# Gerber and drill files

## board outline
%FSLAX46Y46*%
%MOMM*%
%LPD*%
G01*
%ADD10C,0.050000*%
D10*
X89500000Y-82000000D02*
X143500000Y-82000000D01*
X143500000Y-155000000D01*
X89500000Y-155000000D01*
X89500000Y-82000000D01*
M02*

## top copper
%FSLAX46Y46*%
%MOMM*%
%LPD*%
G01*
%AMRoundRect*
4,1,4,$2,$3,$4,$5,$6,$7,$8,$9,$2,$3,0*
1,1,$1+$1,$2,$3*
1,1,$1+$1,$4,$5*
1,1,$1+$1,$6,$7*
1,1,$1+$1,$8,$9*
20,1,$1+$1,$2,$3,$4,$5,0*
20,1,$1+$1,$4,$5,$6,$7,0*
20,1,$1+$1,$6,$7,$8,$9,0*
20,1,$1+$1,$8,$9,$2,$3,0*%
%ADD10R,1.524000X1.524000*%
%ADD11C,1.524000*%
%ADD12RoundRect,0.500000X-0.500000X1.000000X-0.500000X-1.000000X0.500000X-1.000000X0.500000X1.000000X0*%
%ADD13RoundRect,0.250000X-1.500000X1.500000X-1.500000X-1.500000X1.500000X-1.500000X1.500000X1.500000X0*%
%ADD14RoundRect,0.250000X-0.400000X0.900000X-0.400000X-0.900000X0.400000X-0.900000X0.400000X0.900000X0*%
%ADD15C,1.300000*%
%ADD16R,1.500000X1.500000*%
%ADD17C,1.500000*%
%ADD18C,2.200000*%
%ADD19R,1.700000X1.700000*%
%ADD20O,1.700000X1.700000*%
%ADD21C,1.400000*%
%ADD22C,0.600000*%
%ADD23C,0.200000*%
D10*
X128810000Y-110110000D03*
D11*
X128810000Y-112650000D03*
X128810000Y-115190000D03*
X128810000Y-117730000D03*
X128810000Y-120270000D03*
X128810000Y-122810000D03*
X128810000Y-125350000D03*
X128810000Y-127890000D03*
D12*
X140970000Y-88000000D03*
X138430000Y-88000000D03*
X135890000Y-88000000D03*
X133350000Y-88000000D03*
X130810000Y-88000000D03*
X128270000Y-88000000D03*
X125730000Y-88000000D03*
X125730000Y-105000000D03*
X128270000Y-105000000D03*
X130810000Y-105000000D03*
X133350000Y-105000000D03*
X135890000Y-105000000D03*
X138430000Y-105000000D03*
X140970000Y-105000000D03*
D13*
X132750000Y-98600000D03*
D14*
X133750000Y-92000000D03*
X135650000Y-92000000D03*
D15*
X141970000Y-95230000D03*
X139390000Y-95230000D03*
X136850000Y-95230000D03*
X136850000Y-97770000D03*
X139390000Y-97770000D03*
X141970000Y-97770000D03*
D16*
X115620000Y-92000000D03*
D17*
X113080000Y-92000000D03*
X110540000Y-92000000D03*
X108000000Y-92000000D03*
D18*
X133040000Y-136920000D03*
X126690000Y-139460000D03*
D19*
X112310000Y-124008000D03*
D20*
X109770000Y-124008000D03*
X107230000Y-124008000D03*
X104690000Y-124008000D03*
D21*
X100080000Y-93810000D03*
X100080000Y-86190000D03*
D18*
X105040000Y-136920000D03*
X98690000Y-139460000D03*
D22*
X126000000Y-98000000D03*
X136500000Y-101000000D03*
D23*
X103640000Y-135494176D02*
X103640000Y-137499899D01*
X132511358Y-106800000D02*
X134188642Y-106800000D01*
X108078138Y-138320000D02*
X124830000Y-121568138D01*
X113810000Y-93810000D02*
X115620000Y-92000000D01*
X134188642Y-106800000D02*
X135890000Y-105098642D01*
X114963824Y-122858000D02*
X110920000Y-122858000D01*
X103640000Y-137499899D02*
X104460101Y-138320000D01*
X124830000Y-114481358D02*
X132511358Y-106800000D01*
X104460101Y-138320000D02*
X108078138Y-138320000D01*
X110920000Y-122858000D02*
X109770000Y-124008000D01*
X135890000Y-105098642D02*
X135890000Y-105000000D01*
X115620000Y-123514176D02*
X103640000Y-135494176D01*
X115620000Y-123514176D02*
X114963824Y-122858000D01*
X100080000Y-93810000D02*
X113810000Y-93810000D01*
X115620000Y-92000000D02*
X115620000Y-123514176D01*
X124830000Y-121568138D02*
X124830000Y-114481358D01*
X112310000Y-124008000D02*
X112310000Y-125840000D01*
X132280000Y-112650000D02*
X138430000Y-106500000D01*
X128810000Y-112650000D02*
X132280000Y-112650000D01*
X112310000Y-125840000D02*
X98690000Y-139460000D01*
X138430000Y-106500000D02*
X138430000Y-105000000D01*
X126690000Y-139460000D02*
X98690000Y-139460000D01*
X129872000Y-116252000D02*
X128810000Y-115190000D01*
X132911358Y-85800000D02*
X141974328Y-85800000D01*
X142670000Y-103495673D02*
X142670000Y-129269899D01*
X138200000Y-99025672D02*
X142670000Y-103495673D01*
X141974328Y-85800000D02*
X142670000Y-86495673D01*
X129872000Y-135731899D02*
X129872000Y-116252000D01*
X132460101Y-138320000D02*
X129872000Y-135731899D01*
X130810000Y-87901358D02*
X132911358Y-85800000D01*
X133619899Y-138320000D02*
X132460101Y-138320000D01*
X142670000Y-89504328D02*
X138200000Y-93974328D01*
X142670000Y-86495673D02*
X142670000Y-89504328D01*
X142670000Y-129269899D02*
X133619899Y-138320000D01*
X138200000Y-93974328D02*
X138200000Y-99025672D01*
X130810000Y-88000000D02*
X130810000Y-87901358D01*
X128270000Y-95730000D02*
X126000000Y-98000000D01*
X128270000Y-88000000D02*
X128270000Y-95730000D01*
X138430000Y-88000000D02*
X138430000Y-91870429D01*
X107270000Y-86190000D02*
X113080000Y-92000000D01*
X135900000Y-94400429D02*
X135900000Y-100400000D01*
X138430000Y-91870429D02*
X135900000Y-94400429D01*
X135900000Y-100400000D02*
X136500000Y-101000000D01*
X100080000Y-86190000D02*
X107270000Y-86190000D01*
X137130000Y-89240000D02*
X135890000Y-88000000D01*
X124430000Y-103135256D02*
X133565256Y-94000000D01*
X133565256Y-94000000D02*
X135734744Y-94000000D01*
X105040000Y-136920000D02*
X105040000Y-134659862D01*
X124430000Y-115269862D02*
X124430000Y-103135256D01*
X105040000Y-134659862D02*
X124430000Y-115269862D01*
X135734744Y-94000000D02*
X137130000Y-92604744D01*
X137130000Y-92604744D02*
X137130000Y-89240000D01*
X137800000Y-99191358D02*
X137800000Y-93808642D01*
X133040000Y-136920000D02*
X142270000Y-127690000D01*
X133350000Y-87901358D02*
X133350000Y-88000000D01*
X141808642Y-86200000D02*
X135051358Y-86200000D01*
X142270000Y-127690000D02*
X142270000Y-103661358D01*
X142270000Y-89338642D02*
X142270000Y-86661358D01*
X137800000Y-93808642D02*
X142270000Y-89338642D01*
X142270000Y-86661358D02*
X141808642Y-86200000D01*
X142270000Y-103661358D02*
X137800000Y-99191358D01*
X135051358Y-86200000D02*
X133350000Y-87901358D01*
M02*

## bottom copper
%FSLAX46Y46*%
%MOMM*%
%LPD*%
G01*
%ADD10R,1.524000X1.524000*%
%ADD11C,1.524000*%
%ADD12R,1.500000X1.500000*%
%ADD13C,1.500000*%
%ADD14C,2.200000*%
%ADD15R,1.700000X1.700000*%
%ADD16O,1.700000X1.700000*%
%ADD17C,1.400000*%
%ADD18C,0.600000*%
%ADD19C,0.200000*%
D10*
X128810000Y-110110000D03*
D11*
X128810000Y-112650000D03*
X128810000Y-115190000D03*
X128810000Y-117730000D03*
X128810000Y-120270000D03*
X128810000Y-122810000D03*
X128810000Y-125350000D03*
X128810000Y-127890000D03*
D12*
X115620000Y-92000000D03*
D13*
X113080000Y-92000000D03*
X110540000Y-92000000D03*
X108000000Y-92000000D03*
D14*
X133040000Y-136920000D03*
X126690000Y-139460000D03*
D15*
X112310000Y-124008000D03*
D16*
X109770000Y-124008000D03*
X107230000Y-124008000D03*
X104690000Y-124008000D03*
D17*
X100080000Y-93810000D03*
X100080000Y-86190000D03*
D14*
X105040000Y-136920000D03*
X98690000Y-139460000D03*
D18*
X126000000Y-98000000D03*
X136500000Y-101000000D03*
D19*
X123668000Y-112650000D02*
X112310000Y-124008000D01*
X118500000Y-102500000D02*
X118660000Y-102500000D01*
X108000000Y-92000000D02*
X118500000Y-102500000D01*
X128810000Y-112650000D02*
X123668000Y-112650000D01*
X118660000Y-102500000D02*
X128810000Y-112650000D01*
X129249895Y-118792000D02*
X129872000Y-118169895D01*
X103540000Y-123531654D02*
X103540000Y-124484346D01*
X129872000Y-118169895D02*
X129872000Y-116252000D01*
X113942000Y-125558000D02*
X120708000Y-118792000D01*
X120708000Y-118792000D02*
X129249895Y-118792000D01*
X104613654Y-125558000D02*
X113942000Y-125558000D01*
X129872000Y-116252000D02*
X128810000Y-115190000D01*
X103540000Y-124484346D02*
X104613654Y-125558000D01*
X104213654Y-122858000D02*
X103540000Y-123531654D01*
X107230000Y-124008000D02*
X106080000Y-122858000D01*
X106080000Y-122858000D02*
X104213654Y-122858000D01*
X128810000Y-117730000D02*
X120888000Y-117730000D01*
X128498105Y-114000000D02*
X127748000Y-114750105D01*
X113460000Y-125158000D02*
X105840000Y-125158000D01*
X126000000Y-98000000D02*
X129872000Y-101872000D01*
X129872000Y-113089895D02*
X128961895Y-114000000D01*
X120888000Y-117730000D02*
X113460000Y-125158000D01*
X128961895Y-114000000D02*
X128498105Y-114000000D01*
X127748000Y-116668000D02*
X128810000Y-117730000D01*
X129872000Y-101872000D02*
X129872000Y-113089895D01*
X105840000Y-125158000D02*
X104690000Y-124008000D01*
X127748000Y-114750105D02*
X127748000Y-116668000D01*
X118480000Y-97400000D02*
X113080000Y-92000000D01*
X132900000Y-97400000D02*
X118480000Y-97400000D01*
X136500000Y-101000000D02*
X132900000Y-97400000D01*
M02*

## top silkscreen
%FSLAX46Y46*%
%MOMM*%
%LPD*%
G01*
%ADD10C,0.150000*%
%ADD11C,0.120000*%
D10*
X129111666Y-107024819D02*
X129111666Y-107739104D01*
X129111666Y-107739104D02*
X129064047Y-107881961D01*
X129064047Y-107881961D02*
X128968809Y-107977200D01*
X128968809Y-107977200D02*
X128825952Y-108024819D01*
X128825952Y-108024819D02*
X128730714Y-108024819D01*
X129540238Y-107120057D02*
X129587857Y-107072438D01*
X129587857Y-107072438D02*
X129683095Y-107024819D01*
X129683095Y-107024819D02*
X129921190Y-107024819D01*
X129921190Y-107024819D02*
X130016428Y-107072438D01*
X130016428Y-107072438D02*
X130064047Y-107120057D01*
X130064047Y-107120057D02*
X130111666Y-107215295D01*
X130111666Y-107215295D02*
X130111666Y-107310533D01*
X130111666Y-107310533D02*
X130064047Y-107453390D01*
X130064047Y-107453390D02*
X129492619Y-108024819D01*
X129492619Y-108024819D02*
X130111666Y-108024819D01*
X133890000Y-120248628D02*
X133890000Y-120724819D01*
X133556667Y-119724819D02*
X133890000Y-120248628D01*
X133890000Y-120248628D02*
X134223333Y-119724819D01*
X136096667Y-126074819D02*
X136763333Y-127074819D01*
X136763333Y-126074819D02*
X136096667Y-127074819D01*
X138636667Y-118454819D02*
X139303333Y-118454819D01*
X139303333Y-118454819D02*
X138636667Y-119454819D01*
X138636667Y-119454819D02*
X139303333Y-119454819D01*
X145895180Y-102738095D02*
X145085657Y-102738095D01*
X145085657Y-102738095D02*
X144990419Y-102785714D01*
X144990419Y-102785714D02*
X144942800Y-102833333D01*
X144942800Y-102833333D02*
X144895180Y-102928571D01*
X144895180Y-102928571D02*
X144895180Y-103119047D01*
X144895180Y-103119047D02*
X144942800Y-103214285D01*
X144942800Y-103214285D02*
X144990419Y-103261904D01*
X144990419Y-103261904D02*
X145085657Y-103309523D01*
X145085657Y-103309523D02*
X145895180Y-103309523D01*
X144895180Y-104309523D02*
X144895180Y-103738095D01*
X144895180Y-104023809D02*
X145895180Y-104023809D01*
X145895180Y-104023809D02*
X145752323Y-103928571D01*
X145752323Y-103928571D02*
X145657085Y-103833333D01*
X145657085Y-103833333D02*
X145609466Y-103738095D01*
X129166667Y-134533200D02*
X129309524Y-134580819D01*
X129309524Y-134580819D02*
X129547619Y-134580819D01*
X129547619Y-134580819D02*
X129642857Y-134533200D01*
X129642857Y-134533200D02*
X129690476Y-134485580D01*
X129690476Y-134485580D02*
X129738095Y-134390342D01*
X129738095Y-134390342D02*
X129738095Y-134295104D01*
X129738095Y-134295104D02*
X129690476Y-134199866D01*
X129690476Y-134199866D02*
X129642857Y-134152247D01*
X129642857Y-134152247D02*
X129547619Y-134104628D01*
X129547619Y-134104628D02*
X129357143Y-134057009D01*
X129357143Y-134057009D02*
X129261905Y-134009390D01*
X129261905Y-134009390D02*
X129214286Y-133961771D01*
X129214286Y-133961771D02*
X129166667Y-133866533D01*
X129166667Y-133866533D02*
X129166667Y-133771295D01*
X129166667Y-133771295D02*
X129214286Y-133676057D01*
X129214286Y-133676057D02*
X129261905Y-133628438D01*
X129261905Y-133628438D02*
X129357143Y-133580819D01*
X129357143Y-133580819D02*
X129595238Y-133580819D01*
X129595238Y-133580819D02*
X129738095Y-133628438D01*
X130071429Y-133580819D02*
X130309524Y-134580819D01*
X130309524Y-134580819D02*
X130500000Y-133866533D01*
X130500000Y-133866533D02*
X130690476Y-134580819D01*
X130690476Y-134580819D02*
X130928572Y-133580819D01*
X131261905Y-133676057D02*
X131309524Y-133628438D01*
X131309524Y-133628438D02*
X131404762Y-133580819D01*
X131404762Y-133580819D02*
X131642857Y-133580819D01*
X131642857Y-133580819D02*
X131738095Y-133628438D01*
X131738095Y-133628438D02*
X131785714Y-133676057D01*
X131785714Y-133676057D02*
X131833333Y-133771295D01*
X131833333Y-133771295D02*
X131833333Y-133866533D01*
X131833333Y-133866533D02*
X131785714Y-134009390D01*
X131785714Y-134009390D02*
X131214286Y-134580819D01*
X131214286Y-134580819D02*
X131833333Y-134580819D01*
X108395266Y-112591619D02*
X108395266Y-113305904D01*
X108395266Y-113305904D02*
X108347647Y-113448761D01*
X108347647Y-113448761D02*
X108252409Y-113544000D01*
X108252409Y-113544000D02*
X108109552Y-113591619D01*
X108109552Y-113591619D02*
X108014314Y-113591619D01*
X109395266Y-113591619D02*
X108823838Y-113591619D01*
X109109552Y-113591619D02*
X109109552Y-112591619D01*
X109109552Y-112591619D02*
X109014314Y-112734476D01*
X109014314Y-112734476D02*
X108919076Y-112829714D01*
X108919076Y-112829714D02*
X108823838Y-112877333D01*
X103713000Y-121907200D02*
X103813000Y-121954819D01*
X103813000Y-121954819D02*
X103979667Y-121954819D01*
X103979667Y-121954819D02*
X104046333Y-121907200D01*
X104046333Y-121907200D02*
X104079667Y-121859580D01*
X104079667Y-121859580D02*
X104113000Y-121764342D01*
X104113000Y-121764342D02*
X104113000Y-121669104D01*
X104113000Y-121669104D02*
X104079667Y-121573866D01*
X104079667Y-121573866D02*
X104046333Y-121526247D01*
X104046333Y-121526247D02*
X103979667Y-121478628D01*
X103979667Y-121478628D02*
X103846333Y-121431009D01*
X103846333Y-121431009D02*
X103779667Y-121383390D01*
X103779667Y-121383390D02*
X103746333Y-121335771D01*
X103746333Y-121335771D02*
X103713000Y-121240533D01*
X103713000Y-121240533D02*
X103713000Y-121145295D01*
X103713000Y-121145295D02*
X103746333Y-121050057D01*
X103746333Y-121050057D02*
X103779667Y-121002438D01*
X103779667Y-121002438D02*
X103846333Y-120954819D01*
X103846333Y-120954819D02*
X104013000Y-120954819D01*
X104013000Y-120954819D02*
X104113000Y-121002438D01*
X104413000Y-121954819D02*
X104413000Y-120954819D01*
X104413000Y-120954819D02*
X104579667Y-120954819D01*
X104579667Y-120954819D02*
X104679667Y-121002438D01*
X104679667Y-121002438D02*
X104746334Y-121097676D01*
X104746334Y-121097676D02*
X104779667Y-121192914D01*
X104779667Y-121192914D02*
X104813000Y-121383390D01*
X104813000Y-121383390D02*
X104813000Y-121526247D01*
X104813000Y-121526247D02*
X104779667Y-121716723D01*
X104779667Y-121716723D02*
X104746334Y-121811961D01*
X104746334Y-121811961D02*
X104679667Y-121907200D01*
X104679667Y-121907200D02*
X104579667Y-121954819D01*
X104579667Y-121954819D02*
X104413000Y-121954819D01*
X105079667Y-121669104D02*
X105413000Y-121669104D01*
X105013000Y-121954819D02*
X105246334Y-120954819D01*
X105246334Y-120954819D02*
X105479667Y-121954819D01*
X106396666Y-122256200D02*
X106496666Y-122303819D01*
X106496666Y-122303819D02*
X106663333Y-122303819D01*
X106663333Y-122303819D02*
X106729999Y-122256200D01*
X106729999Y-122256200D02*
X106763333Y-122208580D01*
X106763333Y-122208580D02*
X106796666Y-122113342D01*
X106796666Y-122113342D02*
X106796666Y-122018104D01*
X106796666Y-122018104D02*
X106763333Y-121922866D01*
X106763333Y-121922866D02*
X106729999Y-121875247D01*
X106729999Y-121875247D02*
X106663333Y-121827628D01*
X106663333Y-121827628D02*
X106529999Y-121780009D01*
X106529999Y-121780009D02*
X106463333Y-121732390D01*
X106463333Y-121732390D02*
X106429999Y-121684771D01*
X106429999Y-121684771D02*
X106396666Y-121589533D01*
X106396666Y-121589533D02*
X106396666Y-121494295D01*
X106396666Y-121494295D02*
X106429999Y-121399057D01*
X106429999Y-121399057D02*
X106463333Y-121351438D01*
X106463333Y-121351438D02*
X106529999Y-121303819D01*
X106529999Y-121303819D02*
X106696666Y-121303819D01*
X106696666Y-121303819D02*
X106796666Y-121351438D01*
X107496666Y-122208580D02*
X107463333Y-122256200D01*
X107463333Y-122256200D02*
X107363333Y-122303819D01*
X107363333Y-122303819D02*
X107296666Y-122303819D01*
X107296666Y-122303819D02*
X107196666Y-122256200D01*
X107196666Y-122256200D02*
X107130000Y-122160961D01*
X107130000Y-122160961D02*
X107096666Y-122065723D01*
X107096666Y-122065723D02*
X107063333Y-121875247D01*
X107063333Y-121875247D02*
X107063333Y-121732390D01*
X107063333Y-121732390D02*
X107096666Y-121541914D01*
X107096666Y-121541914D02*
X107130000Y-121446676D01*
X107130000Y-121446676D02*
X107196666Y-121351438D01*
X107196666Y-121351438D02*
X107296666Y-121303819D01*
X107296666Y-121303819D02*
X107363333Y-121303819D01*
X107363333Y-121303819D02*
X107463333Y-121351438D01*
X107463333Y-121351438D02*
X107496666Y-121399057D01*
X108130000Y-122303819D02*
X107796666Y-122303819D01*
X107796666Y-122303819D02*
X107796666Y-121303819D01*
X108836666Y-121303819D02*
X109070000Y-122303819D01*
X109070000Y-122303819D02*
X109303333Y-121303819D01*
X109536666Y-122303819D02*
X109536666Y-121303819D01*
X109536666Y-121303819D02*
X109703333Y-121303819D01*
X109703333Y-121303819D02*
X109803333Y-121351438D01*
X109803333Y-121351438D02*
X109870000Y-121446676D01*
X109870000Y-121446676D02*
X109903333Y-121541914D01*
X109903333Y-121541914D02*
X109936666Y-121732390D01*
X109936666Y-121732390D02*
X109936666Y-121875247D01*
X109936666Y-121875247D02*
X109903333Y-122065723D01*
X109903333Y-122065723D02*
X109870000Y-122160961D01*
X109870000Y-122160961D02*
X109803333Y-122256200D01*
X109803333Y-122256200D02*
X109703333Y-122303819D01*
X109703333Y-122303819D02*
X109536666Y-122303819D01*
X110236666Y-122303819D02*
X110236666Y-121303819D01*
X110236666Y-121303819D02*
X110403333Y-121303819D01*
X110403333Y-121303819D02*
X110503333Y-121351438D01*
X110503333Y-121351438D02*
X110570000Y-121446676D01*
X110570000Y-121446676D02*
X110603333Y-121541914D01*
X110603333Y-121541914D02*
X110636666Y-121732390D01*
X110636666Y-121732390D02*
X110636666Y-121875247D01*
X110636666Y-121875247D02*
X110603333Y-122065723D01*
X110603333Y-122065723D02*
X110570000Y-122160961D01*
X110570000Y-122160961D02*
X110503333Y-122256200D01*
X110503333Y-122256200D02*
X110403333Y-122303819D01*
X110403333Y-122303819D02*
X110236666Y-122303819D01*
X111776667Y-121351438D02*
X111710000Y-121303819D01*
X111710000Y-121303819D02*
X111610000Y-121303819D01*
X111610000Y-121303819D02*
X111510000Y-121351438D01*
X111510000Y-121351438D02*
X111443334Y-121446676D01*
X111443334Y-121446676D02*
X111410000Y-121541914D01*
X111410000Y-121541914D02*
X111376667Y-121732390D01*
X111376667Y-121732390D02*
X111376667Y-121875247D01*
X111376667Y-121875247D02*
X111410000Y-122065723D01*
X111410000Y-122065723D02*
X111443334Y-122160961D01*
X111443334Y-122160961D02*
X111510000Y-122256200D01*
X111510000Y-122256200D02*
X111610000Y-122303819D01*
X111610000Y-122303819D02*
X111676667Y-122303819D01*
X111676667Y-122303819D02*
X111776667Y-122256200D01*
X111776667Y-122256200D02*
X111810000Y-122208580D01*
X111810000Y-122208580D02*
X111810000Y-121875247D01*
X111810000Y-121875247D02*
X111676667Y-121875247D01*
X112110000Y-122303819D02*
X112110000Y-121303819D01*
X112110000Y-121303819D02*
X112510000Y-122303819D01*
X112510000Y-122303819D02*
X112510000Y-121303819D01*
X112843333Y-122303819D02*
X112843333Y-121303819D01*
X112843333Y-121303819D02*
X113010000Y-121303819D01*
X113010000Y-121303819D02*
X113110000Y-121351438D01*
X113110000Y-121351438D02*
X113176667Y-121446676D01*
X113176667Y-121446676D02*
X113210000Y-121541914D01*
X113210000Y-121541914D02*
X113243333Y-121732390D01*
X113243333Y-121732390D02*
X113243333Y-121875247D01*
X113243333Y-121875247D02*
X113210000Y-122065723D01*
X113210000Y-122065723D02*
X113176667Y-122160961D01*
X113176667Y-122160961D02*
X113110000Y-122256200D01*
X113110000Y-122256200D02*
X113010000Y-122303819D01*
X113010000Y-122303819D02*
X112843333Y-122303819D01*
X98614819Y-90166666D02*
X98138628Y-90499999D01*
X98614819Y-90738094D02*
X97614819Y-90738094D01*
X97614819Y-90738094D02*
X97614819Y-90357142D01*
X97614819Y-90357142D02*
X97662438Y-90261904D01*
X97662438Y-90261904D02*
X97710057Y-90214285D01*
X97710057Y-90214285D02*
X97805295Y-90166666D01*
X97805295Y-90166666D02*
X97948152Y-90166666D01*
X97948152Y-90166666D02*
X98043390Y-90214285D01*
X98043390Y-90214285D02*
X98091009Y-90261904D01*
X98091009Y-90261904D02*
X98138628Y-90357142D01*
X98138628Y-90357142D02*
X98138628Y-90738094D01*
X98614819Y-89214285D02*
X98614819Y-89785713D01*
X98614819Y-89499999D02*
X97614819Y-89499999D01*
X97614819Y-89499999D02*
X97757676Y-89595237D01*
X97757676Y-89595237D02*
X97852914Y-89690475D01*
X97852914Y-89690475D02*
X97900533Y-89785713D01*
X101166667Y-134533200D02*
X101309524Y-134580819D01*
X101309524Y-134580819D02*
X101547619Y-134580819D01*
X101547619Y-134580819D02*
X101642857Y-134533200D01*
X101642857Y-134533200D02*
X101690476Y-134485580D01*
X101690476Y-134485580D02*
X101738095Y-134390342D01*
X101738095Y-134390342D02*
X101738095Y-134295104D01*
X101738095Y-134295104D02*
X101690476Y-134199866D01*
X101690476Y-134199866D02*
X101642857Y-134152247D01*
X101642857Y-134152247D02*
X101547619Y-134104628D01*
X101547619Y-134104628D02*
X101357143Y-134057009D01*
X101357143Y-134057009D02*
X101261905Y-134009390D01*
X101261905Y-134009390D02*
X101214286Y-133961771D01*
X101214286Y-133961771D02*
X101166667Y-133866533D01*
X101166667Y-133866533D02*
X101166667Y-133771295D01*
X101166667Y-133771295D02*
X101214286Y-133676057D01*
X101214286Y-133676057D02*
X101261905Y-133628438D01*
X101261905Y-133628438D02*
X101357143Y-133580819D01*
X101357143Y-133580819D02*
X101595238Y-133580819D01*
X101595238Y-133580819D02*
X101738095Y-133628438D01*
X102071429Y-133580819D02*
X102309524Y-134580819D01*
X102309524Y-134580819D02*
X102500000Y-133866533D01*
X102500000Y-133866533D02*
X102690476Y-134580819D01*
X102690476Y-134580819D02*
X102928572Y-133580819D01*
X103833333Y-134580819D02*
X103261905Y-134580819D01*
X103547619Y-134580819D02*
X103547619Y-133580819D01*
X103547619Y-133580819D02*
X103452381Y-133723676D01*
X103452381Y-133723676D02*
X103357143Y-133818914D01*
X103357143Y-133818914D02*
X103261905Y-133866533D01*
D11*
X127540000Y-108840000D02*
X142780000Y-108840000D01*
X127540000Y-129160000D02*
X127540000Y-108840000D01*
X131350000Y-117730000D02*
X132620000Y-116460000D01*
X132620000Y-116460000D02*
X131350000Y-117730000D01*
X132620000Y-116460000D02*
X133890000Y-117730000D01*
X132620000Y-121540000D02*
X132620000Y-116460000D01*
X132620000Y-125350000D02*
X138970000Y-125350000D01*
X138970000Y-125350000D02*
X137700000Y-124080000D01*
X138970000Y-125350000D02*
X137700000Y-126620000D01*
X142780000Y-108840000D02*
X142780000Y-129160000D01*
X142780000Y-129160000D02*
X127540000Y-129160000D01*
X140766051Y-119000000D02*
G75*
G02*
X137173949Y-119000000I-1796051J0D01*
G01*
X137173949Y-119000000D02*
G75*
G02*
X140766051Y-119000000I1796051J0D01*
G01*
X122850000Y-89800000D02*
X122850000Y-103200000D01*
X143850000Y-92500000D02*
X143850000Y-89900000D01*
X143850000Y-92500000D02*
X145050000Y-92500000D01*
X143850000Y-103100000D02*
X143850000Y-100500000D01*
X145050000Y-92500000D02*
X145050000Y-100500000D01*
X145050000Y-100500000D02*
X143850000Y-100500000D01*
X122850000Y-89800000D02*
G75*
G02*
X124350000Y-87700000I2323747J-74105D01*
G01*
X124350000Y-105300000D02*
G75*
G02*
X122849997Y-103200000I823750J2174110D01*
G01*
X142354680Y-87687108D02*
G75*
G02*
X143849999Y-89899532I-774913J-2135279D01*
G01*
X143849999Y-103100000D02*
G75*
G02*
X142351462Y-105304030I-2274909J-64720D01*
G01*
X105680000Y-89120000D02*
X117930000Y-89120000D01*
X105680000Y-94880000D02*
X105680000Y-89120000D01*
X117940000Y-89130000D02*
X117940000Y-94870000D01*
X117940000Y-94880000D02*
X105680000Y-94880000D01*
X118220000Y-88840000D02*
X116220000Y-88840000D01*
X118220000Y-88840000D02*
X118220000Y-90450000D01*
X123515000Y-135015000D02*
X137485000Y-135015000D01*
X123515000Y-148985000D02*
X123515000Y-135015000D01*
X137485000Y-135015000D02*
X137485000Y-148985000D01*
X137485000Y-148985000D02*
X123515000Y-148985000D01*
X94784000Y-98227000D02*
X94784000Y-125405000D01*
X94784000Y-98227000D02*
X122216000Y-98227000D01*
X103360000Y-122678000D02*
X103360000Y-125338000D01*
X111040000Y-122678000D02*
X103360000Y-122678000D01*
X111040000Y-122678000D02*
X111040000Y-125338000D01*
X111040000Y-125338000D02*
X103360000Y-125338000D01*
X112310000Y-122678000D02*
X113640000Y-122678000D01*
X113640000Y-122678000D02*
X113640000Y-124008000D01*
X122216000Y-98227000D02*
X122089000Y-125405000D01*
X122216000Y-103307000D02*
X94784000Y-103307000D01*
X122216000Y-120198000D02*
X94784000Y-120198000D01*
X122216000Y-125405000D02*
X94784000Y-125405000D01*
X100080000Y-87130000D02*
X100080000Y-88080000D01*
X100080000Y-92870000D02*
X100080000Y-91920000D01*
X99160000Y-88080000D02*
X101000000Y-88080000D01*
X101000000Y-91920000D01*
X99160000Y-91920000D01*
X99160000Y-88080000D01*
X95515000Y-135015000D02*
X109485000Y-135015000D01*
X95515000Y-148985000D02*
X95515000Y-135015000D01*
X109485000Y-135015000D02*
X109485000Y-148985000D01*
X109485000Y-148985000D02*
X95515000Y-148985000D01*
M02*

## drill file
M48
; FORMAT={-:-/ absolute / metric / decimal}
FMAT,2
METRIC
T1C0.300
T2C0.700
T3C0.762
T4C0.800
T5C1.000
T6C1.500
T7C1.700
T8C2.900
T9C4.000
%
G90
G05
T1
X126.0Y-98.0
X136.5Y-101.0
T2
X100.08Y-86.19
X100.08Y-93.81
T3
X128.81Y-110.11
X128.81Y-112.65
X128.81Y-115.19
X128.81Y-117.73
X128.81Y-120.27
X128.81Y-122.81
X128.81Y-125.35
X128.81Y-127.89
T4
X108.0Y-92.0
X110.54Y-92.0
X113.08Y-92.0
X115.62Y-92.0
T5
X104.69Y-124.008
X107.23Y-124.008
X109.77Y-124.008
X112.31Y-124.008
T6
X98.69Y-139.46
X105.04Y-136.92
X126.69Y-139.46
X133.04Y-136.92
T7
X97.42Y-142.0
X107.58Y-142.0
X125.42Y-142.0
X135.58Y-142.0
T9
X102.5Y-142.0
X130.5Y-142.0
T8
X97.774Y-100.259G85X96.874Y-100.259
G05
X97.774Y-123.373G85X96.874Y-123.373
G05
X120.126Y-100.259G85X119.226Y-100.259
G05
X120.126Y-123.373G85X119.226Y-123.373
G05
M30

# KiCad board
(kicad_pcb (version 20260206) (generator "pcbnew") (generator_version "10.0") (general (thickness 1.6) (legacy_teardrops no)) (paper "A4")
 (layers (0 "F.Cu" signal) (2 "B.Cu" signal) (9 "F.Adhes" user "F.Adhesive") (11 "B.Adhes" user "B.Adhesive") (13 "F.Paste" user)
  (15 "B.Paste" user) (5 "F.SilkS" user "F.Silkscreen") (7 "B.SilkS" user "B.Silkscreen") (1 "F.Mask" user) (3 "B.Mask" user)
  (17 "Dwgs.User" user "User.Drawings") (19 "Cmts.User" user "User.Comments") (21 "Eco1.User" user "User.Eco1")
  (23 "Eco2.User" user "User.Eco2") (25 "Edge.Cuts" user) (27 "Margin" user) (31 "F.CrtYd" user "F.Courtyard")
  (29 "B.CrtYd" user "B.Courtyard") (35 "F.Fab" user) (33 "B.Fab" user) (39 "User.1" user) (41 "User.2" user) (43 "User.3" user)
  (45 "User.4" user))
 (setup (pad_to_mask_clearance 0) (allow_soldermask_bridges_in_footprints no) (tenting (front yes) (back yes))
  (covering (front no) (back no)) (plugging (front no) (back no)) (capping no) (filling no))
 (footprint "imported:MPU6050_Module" (layer "F.Cu") (at 128.81 110.11)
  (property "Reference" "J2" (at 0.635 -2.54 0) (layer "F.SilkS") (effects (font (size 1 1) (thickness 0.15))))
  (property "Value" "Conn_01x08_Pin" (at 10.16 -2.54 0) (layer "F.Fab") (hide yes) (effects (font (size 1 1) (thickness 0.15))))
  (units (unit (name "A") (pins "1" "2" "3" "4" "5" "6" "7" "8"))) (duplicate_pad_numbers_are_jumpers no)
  (fp_line (start -1.27 -1.27) (end 13.97 -1.27) (stroke (width 0.12) (type solid)) (layer "F.SilkS"))
  (fp_line (start -1.27 19.05) (end -1.27 -1.27) (stroke (width 0.12) (type solid)) (layer "F.SilkS"))
  (fp_line (start 2.54 7.62) (end 3.81 6.35) (stroke (width 0.12) (type solid)) (layer "F.SilkS"))
  (fp_line (start 3.81 6.35) (end 2.54 7.62) (stroke (width 0.12) (type solid)) (layer "F.SilkS"))
  (fp_line (start 3.81 6.35) (end 5.08 7.62) (stroke (width 0.12) (type solid)) (layer "F.SilkS"))
  (fp_line (start 3.81 11.43) (end 3.81 6.35) (stroke (width 0.12) (type solid)) (layer "F.SilkS"))
  (fp_line (start 3.81 15.24) (end 10.16 15.24) (stroke (width 0.12) (type solid)) (layer "F.SilkS"))
  (fp_line (start 10.16 15.24) (end 8.89 13.97) (stroke (width 0.12) (type solid)) (layer "F.SilkS"))
  (fp_line (start 10.16 15.24) (end 8.89 16.51) (stroke (width 0.12) (type solid)) (layer "F.SilkS"))
  (fp_line (start 13.97 -1.27) (end 13.97 19.05) (stroke (width 0.12) (type solid)) (layer "F.SilkS"))
  (fp_line (start 13.97 19.05) (end -1.27 19.05) (stroke (width 0.12) (type solid)) (layer "F.SilkS"))
  (fp_circle (center 10.16 8.89) (end 8.89 7.62) (stroke (width 0.12) (type solid)) (fill no) (layer "F.SilkS"))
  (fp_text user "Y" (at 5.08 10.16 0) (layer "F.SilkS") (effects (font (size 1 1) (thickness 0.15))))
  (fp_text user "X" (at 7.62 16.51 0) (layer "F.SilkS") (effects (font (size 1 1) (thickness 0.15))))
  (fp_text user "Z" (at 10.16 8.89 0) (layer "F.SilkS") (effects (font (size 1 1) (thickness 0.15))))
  (pad "1" thru_hole rect (at 0 0) (size 1.524 1.524) (drill 0.762) (layers "*.Cu" "*.Mask") (remove_unused_layers no) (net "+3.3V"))
  (pad "2" thru_hole circle (at 0 2.54) (size 1.524 1.524) (drill 0.762) (layers "*.Cu" "*.Mask") (remove_unused_layers no) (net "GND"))
  (pad "3" thru_hole circle (at 0 5.08) (size 1.524 1.524) (drill 0.762) (layers "*.Cu" "*.Mask") (remove_unused_layers no) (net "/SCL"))
  (pad "4" thru_hole circle (at 0 7.62) (size 1.524 1.524) (drill 0.762) (layers "*.Cu" "*.Mask") (remove_unused_layers no) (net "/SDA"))
  (pad "5" thru_hole circle (at 0 10.16) (size 1.524 1.524) (drill 0.762) (layers "*.Cu" "*.Mask") (remove_unused_layers no)
   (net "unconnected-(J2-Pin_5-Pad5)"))
  (pad "6" thru_hole circle (at 0 12.7) (size 1.524 1.524) (drill 0.762) (layers "*.Cu" "*.Mask") (remove_unused_layers no)
   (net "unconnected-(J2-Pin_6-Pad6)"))
  (pad "7" thru_hole circle (at 0 15.24) (size 1.524 1.524) (drill 0.762) (layers "*.Cu" "*.Mask") (remove_unused_layers no)
   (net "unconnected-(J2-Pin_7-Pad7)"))
  (pad "8" thru_hole circle (at 0 17.78) (size 1.524 1.524) (drill 0.762) (layers "*.Cu" "*.Mask") (remove_unused_layers no)
   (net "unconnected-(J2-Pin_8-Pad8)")))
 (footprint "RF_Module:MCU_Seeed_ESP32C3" (layer "F.Cu") (at 133.35 96.5 -90)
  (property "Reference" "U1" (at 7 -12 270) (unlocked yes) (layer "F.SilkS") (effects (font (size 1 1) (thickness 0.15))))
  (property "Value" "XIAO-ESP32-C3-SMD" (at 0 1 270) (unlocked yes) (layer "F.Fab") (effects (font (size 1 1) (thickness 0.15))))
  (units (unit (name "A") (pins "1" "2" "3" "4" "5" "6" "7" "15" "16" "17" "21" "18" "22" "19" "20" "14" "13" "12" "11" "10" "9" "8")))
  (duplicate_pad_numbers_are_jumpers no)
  (fp_line (start -6.7 10.5) (end 6.7 10.5) (stroke (width 0.12) (type default)) (layer "F.SilkS"))
  (fp_line (start -4 -10.5) (end -6.6 -10.5) (stroke (width 0.12) (type default)) (layer "F.SilkS"))
  (fp_line (start -4 -10.5) (end -4 -11.7) (stroke (width 0.12) (type default)) (layer "F.SilkS"))
  (fp_line (start 6.6 -10.5) (end 4 -10.5) (stroke (width 0.12) (type default)) (layer "F.SilkS"))
  (fp_line (start -4 -11.7) (end 4 -11.7) (stroke (width 0.12) (type default)) (layer "F.SilkS"))
  (fp_line (start 4 -11.7) (end 4 -10.5) (stroke (width 0.12) (type default)) (layer "F.SilkS"))
  (fp_arc (start -6.7 10.5) (mid -7.977232 10.068125) (end -8.8 9) (stroke (width 0.12) (type default)) (layer "F.SilkS"))
  (fp_arc (start 8.8 9) (mid 7.977232 10.068125) (end 6.7 10.5) (stroke (width 0.12) (type default)) (layer "F.SilkS"))
  (fp_arc (start -8.812892 -9.00468) (mid -7.949609 -10.111769) (end -6.600468 -10.499999) (stroke (width 0.12) (type default))
   (layer "F.SilkS"))
  (fp_arc (start 6.6 -10.499999) (mid 7.944325 -10.107116) (end 8.804034 -9.001464) (stroke (width 0.12) (type default)) (layer "F.SilkS"))
  (pad "" smd roundrect (at 1.1 -0.4 270) (size 1.5 1.5) (layers "F.Paste") (roundrect_rratio 0.1666666667))
  (pad "" smd roundrect (at 1.1 1.6 270) (size 1.5 1.5) (layers "F.Paste") (roundrect_rratio 0.1666666667))
  (pad "" smd roundrect (at 3.1 -0.4 270) (size 1.5 1.5) (layers "F.Paste") (roundrect_rratio 0.1666666667))
  (pad "" smd roundrect (at 3.1 1.6 270) (size 1.5 1.5) (layers "F.Paste") (roundrect_rratio 0.1666666667))
  (pad "1" smd roundrect (at -8.5 -7.62 270) (size 3 2) (layers "F.Cu" "F.Mask" "F.Paste") (roundrect_rratio 0.25)
   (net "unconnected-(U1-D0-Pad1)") (thermal_bridge_angle 45))
  (pad "2" smd roundrect (at -8.5 -5.08 270) (size 3 2) (layers "F.Cu" "F.Mask" "F.Paste") (roundrect_rratio 0.25) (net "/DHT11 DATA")
   (thermal_bridge_angle 45))
  (pad "3" smd roundrect (at -8.5 -2.54 270) (size 3 2) (layers "F.Cu" "F.Mask" "F.Paste") (roundrect_rratio 0.25) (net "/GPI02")
   (thermal_bridge_angle 45))
  (pad "4" smd roundrect (at -8.5 0 270) (size 3 2) (layers "F.Cu" "F.Mask" "F.Paste") (roundrect_rratio 0.25) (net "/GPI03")
   (thermal_bridge_angle 45))
  (pad "5" smd roundrect (at -8.5 2.54 270) (size 3 2) (layers "F.Cu" "F.Mask" "F.Paste") (roundrect_rratio 0.25) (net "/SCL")
   (thermal_bridge_angle 45))
  (pad "6" smd roundrect (at -8.5 5.08 270) (size 3 2) (layers "F.Cu" "F.Mask" "F.Paste") (roundrect_rratio 0.25) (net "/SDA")
   (thermal_bridge_angle 45))
  (pad "7" smd roundrect (at -8.5 7.62 270) (size 3 2) (layers "F.Cu" "F.Mask" "F.Paste") (roundrect_rratio 0.25)
   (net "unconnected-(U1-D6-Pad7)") (thermal_bridge_angle 45))
  (pad "8" smd roundrect (at 8.5 7.62 270) (size 3 2) (layers "F.Cu" "F.Mask" "F.Paste") (roundrect_rratio 0.25)
   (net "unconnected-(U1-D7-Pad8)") (thermal_bridge_angle 45))
  (pad "9" smd roundrect (at 8.5 5.08 270) (size 3 2) (layers "F.Cu" "F.Mask" "F.Paste") (roundrect_rratio 0.25)
   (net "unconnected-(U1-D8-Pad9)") (thermal_bridge_angle 45))
  (pad "10" smd roundrect (at 8.5 2.54 270) (size 3 2) (layers "F.Cu" "F.Mask" "F.Paste") (roundrect_rratio 0.25)
   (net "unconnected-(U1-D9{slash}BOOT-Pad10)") (thermal_bridge_angle 45))
  (pad "11" smd roundrect (at 8.5 0 270) (size 3 2) (layers "F.Cu" "F.Mask" "F.Paste") (roundrect_rratio 0.25)
   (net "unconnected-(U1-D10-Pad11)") (thermal_bridge_angle 45))
  (pad "12" smd roundrect (at 8.5 -2.54 270) (size 3 2) (layers "F.Cu" "F.Mask" "F.Paste") (roundrect_rratio 0.25) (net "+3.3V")
   (thermal_bridge_angle 45))
  (pad "13" smd roundrect (at 8.5 -5.08 270) (size 3 2) (layers "F.Cu" "F.Mask" "F.Paste") (roundrect_rratio 0.25) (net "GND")
   (thermal_bridge_angle 45))
  (pad "14" smd roundrect (at 8.5 -7.62 270) (size 3 2) (layers "F.Cu" "F.Mask" "F.Paste") (roundrect_rratio 0.25) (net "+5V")
   (thermal_bridge_angle 45))
  (pad "15" smd roundrect (at 2.1 0.6 270) (size 3.5 3.5) (layers "F.Cu" "F.Mask") (roundrect_rratio 0.07142857143)
   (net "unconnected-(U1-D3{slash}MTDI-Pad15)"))
  (pad "16" smd roundrect (at -4.5 -0.4 270) (size 2.3 1.3) (layers "F.Cu" "F.Mask" "F.Paste") (roundrect_rratio 0.1923076923)
   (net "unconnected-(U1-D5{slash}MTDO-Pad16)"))
  (pad "17" smd roundrect (at -4.5 -2.3 270) (size 2.3 1.3) (layers "F.Cu" "F.Mask" "F.Paste") (roundrect_rratio 0.1923076923)
   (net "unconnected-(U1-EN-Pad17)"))
  (pad "18" smd circle (at -1.27 -8.62 270) (size 1.3 1.3) (layers "F.Cu" "F.Mask" "F.Paste") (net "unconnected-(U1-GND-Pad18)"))
  (pad "19" smd circle (at -1.27 -6.04 270) (size 1.3 1.3) (layers "F.Cu" "F.Mask" "F.Paste") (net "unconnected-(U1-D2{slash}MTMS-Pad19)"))
  (pad "20" smd circle (at -1.27 -3.5 270) (size 1.3 1.3) (layers "F.Cu" "F.Mask" "F.Paste") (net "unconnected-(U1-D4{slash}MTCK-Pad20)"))
  (pad "21" smd circle (at 1.27 -3.5 270) (size 1.3 1.3) (layers "F.Cu" "F.Mask" "F.Paste") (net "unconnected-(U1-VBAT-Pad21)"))
  (pad "22" smd circle (at 1.27 -6.04 270) (size 1.3 1.3) (layers "F.Cu" "F.Mask" "F.Paste") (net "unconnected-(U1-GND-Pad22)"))
  (pad "23" smd circle (at 1.27 -8.62 270) (size 1.3 1.3) (layers "F.Cu" "F.Mask" "F.Paste")))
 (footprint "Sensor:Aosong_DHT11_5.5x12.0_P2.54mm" (layer "F.Cu") (at 115.62 92 -90)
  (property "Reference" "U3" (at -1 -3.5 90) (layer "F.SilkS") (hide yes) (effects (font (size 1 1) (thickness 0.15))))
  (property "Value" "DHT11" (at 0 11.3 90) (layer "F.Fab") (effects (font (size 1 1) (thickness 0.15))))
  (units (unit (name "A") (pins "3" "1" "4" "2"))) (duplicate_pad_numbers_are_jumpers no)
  (fp_line (start -2.88 9.94) (end -2.88 -2.31) (stroke (width 0.12) (type solid)) (layer "F.SilkS"))
  (fp_line (start 2.88 9.94) (end -2.88 9.94) (stroke (width 0.12) (type solid)) (layer "F.SilkS"))
  (fp_line (start -2.87 -2.32) (end 2.87 -2.32) (stroke (width 0.12) (type solid)) (layer "F.SilkS"))
  (fp_line (start 2.88 -2.32) (end 2.88 9.94) (stroke (width 0.12) (type solid)) (layer "F.SilkS"))
  (fp_line (start -3.16 -2.6) (end -3.16 -0.6) (stroke (width 0.12) (type solid)) (layer "F.SilkS"))
  (fp_line (start -3.16 -2.6) (end -1.55 -2.6) (stroke (width 0.12) (type solid)) (layer "F.SilkS"))
  (pad "1" thru_hole rect (at 0 0 270) (size 1.5 1.5) (drill 0.8) (layers "*.Cu" "*.Mask") (remove_unused_layers no) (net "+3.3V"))
  (pad "2" thru_hole circle (at 0 2.54 270) (size 1.5 1.5) (drill 0.8) (layers "*.Cu" "*.Mask") (remove_unused_layers no)
   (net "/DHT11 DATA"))
  (pad "3" thru_hole circle (at 0 5.08 270) (size 1.5 1.5) (drill 0.8) (layers "*.Cu" "*.Mask") (remove_unused_layers no)
   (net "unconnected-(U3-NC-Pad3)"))
  (pad "4" thru_hole circle (at 0 7.62 270) (size 1.5 1.5) (drill 0.8) (layers "*.Cu" "*.Mask") (remove_unused_layers no) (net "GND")))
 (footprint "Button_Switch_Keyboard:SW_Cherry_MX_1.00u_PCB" (layer "F.Cu") (at 133.04 136.92)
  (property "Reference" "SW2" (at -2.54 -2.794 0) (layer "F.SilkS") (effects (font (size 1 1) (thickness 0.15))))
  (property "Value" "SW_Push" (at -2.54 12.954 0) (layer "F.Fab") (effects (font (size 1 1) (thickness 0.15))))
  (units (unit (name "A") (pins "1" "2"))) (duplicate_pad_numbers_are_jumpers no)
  (fp_line (start -9.525 -1.905) (end 4.445 -1.905) (stroke (width 0.12) (type solid)) (layer "F.SilkS"))
  (fp_line (start -9.525 12.065) (end -9.525 -1.905) (stroke (width 0.12) (type solid)) (layer "F.SilkS"))
  (fp_line (start 4.445 -1.905) (end 4.445 12.065) (stroke (width 0.12) (type solid)) (layer "F.SilkS"))
  (fp_line (start 4.445 12.065) (end -9.525 12.065) (stroke (width 0.12) (type solid)) (layer "F.SilkS"))
  (pad "" np_thru_hole circle (at -7.62 5.08) (size 1.7 1.7) (drill 1.7) (layers "*.Cu" "*.Mask"))
  (pad "" np_thru_hole circle (at -2.54 5.08) (size 4 4) (drill 4) (layers "*.Cu" "*.Mask"))
  (pad "" np_thru_hole circle (at 2.54 5.08) (size 1.7 1.7) (drill 1.7) (layers "*.Cu" "*.Mask"))
  (pad "1" thru_hole circle (at 0 0) (size 2.2 2.2) (drill 1.5) (layers "*.Cu" "*.Mask") (remove_unused_layers no) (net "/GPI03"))
  (pad "2" thru_hole circle (at -6.35 2.54) (size 2.2 2.2) (drill 1.5) (layers "*.Cu" "*.Mask") (remove_unused_layers no) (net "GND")))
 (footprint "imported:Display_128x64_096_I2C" (layer "F.Cu") (at 108.5 124.008 180)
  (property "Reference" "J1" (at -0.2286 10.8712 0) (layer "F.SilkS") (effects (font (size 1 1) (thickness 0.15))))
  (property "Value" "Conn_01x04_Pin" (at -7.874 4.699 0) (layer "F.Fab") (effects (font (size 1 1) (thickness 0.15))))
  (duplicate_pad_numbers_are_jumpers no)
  (fp_line (start 13.716 25.781) (end 13.716 -1.397) (stroke (width 0.12) (type solid)) (layer "F.SilkS"))
  (fp_line (start 13.716 25.781) (end -13.716 25.781) (stroke (width 0.12) (type solid)) (layer "F.SilkS"))
  (fp_line (start 5.14 1.33) (end 5.14 -1.33) (stroke (width 0.12) (type solid)) (layer "F.SilkS"))
  (fp_line (start -2.54 1.33) (end 5.14 1.33) (stroke (width 0.12) (type solid)) (layer "F.SilkS"))
  (fp_line (start -2.54 1.33) (end -2.54 -1.33) (stroke (width 0.12) (type solid)) (layer "F.SilkS"))
  (fp_line (start -2.54 -1.33) (end 5.14 -1.33) (stroke (width 0.12) (type solid)) (layer "F.SilkS"))
  (fp_line (start -3.81 1.33) (end -5.14 1.33) (stroke (width 0.12) (type solid)) (layer "F.SilkS"))
  (fp_line (start -5.14 1.33) (end -5.14 0) (stroke (width 0.12) (type solid)) (layer "F.SilkS"))
  (fp_line (start -13.716 25.781) (end -13.589 -1.397) (stroke (width 0.12) (type solid)) (layer "F.SilkS"))
  (fp_line (start -13.716 20.701) (end 13.716 20.701) (stroke (width 0.12) (type solid)) (layer "F.SilkS"))
  (fp_line (start -13.716 3.81) (end 13.716 3.81) (stroke (width 0.12) (type solid)) (layer "F.SilkS"))
  (fp_line (start -13.716 -1.397) (end 13.716 -1.397) (stroke (width 0.12) (type solid)) (layer "F.SilkS"))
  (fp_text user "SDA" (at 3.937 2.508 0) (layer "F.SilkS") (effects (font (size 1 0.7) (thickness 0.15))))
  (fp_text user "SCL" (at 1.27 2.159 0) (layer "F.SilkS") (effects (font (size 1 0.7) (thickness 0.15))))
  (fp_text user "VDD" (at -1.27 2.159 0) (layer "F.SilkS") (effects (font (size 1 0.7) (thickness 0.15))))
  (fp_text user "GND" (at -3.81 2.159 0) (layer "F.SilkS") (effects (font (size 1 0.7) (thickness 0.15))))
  (pad "" np_thru_hole oval (at -11.176 0.635 180) (size 3.8 2.9) (drill oval 3.8 2.9) (layers "*.Cu" "*.Mask"))
  (pad "" np_thru_hole oval (at -11.176 23.749 180) (size 3.8 2.9) (drill oval 3.8 2.9) (layers "*.Cu" "*.Mask"))
  (pad "" np_thru_hole oval (at 11.176 0.635 180) (size 3.8 2.9) (drill oval 3.8 2.9) (layers "*.Cu" "*.Mask"))
  (pad "" np_thru_hole oval (at 11.176 23.749 180) (size 3.8 2.9) (drill oval 3.8 2.9) (layers "*.Cu" "*.Mask"))
  (pad "1" thru_hole rect (at -3.81 0 270) (size 1.7 1.7) (drill 1) (layers "*.Cu" "*.Mask") (remove_unused_layers no) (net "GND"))
  (pad "2" thru_hole oval (at -1.27 0 270) (size 1.7 1.7) (drill 1) (layers "*.Cu" "*.Mask") (remove_unused_layers no) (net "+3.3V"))
  (pad "3" thru_hole oval (at 1.27 0 270) (size 1.7 1.7) (drill 1) (layers "*.Cu" "*.Mask") (remove_unused_layers no) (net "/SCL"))
  (pad "4" thru_hole oval (at 3.81 0 270) (size 1.7 1.7) (drill 1) (layers "*.Cu" "*.Mask") (remove_unused_layers no) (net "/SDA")))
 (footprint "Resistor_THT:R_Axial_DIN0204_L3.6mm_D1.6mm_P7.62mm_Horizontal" (layer "F.Cu") (at 100.08 93.81 90)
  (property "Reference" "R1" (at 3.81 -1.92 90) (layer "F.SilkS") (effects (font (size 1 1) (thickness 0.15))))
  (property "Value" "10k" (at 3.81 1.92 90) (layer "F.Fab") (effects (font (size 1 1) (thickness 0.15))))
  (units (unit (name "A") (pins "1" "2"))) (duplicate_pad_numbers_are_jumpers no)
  (fp_line (start 6.68 0) (end 5.73 0) (stroke (width 0.12) (type solid)) (layer "F.SilkS"))
  (fp_line (start 0.94 0) (end 1.89 0) (stroke (width 0.12) (type solid)) (layer "F.SilkS"))
  (fp_rect (start 1.89 -0.92) (end 5.73 0.92) (stroke (width 0.12) (type solid)) (fill no) (layer "F.SilkS"))
  (pad "1" thru_hole circle (at 0 0 90) (size 1.4 1.4) (drill 0.7) (layers "*.Cu" "*.Mask") (remove_unused_layers no) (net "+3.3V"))
  (pad "2" thru_hole circle (at 7.62 0 90) (size 1.4 1.4) (drill 0.7) (layers "*.Cu" "*.Mask") (remove_unused_layers no) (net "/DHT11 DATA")))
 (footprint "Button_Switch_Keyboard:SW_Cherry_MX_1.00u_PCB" (layer "F.Cu") (at 105.04 136.92)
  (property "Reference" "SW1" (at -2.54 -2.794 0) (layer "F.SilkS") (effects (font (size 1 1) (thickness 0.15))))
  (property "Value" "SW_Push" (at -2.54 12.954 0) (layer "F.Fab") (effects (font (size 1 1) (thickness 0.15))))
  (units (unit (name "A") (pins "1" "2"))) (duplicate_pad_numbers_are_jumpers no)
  (fp_line (start -9.525 -1.905) (end 4.445 -1.905) (stroke (width 0.12) (type solid)) (layer "F.SilkS"))
  (fp_line (start -9.525 12.065) (end -9.525 -1.905) (stroke (width 0.12) (type solid)) (layer "F.SilkS"))
  (fp_line (start 4.445 -1.905) (end 4.445 12.065) (stroke (width 0.12) (type solid)) (layer "F.SilkS"))
  (fp_line (start 4.445 12.065) (end -9.525 12.065) (stroke (width 0.12) (type solid)) (layer "F.SilkS"))
  (pad "" np_thru_hole circle (at -7.62 5.08) (size 1.7 1.7) (drill 1.7) (layers "*.Cu" "*.Mask"))
  (pad "" np_thru_hole circle (at -2.54 5.08) (size 4 4) (drill 4) (layers "*.Cu" "*.Mask"))
  (pad "" np_thru_hole circle (at 2.54 5.08) (size 1.7 1.7) (drill 1.7) (layers "*.Cu" "*.Mask"))
  (pad "1" thru_hole circle (at 0 0) (size 2.2 2.2) (drill 1.5) (layers "*.Cu" "*.Mask") (remove_unused_layers no) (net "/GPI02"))
  (pad "2" thru_hole circle (at -6.35 2.54) (size 2.2 2.2) (drill 1.5) (layers "*.Cu" "*.Mask") (remove_unused_layers no) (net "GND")))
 (gr_rect (start 89.5 82) (end 143.5 155) (stroke (width 0.05) (type default)) (fill no) (layer "Edge.Cuts"))
 (segment (start 103.64 135.494176) (end 103.64 137.499899) (width 0.2) (layer "F.Cu") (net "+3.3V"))
 (segment (start 132.511358 106.8) (end 134.188642 106.8) (width 0.2) (layer "F.Cu") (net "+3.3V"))
 (segment (start 108.078138 138.32) (end 124.83 121.568138) (width 0.2) (layer "F.Cu") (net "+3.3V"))
 (segment (start 113.81 93.81) (end 115.62 92) (width 0.2) (layer "F.Cu") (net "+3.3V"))
 (segment (start 134.188642 106.8) (end 135.89 105.098642) (width 0.2) (layer "F.Cu") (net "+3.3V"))
 (segment (start 114.963824 122.858) (end 110.92 122.858) (width 0.2) (layer "F.Cu") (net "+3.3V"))
 (segment (start 103.64 137.499899) (end 104.460101 138.32) (width 0.2) (layer "F.Cu") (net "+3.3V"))
 (segment (start 124.83 114.481358) (end 132.511358 106.8) (width 0.2) (layer "F.Cu") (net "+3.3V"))
 (segment (start 104.460101 138.32) (end 108.078138 138.32) (width 0.2) (layer "F.Cu") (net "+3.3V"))
 (segment (start 110.92 122.858) (end 109.77 124.008) (width 0.2) (layer "F.Cu") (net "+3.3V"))
 (segment (start 135.89 105.098642) (end 135.89 105) (width 0.2) (layer "F.Cu") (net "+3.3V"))
 (segment (start 115.62 123.514176) (end 103.64 135.494176) (width 0.2) (layer "F.Cu") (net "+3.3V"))
 (segment (start 115.62 123.514176) (end 114.963824 122.858) (width 0.2) (layer "F.Cu") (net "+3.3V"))
 (segment (start 100.08 93.81) (end 113.81 93.81) (width 0.2) (layer "F.Cu") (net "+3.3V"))
 (segment (start 115.62 92) (end 115.62 123.514176) (width 0.2) (layer "F.Cu") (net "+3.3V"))
 (segment (start 124.83 121.568138) (end 124.83 114.481358) (width 0.2) (layer "F.Cu") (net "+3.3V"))
 (segment (start 112.31 124.008) (end 112.31 125.84) (width 0.2) (layer "F.Cu") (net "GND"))
 (segment (start 132.28 112.65) (end 138.43 106.5) (width 0.2) (layer "F.Cu") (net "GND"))
 (segment (start 128.81 112.65) (end 132.28 112.65) (width 0.2) (layer "F.Cu") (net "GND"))
 (segment (start 112.31 125.84) (end 98.69 139.46) (width 0.2) (layer "F.Cu") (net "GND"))
 (segment (start 138.43 106.5) (end 138.43 105) (width 0.2) (layer "F.Cu") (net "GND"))
 (segment (start 126.69 139.46) (end 98.69 139.46) (width 0.2) (layer "F.Cu") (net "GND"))
 (segment (start 123.668 112.65) (end 112.31 124.008) (width 0.2) (layer "B.Cu") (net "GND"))
 (segment (start 118.5 102.5) (end 118.66 102.5) (width 0.2) (layer "B.Cu") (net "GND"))
 (segment (start 108 92) (end 118.5 102.5) (width 0.2) (layer "B.Cu") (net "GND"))
 (segment (start 128.81 112.65) (end 123.668 112.65) (width 0.2) (layer "B.Cu") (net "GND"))
 (segment (start 118.66 102.5) (end 128.81 112.65) (width 0.2) (layer "B.Cu") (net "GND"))
 (segment (start 129.872 116.252) (end 128.81 115.19) (width 0.2) (layer "F.Cu") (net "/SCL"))
 (segment (start 132.911358 85.8) (end 141.974328 85.8) (width 0.2) (layer "F.Cu") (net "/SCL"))
 (segment (start 142.67 103.495673) (end 142.67 129.269899) (width 0.2) (layer "F.Cu") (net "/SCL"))
 (segment (start 138.2 99.025672) (end 142.67 103.495673) (width 0.2) (layer "F.Cu") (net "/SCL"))
 (segment (start 141.974328 85.8) (end 142.67 86.495673) (width 0.2) (layer "F.Cu") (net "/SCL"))
 (segment (start 129.872 135.731899) (end 129.872 116.252) (width 0.2) (layer "F.Cu") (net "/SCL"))
 (segment (start 132.460101 138.32) (end 129.872 135.731899) (width 0.2) (layer "F.Cu") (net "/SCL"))
 (segment (start 130.81 87.901358) (end 132.911358 85.8) (width 0.2) (layer "F.Cu") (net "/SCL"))
 (segment (start 133.619899 138.32) (end 132.460101 138.32) (width 0.2) (layer "F.Cu") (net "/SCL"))
 (segment (start 142.67 89.504328) (end 138.2 93.974328) (width 0.2) (layer "F.Cu") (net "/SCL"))
 (segment (start 142.67 86.495673) (end 142.67 89.504328) (width 0.2) (layer "F.Cu") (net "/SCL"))
 (segment (start 142.67 129.269899) (end 133.619899 138.32) (width 0.2) (layer "F.Cu") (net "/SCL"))
 (segment (start 138.2 93.974328) (end 138.2 99.025672) (width 0.2) (layer "F.Cu") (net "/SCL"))
 (segment (start 130.81 88) (end 130.81 87.901358) (width 0.2) (layer "F.Cu") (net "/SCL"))
 (segment (start 129.249895 118.792) (end 129.872 118.169895) (width 0.2) (layer "B.Cu") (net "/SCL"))
 (segment (start 103.54 123.531654) (end 103.54 124.484346) (width 0.2) (layer "B.Cu") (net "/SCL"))
 (segment (start 129.872 118.169895) (end 129.872 116.252) (width 0.2) (layer "B.Cu") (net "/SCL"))
 (segment (start 113.942 125.558) (end 120.708 118.792) (width 0.2) (layer "B.Cu") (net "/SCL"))
 (segment (start 120.708 118.792) (end 129.249895 118.792) (width 0.2) (layer "B.Cu") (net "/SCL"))
 (segment (start 104.613654 125.558) (end 113.942 125.558) (width 0.2) (layer "B.Cu") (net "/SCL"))
 (segment (start 129.872 116.252) (end 128.81 115.19) (width 0.2) (layer "B.Cu") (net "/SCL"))
 (segment (start 103.54 124.484346) (end 104.613654 125.558) (width 0.2) (layer "B.Cu") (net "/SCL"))
 (segment (start 104.213654 122.858) (end 103.54 123.531654) (width 0.2) (layer "B.Cu") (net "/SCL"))
 (segment (start 107.23 124.008) (end 106.08 122.858) (width 0.2) (layer "B.Cu") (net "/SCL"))
 (segment (start 106.08 122.858) (end 104.213654 122.858) (width 0.2) (layer "B.Cu") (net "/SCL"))
 (segment (start 128.27 95.73) (end 126 98) (width 0.2) (layer "F.Cu") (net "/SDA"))
 (segment (start 128.27 88) (end 128.27 95.73) (width 0.2) (layer "F.Cu") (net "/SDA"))
 (via (at 126 98) (size 0.6) (drill 0.3) (layers "F.Cu" "B.Cu") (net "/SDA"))
 (segment (start 128.81 117.73) (end 120.888 117.73) (width 0.2) (layer "B.Cu") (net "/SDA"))
 (segment (start 128.498105 114) (end 127.748 114.750105) (width 0.2) (layer "B.Cu") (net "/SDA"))
 (segment (start 113.46 125.158) (end 105.84 125.158) (width 0.2) (layer "B.Cu") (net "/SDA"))
 (segment (start 126 98) (end 129.872 101.872) (width 0.2) (layer "B.Cu") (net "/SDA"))
 (segment (start 129.872 113.089895) (end 128.961895 114) (width 0.2) (layer "B.Cu") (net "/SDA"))
 (segment (start 120.888 117.73) (end 113.46 125.158) (width 0.2) (layer "B.Cu") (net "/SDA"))
 (segment (start 128.961895 114) (end 128.498105 114) (width 0.2) (layer "B.Cu") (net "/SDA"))
 (segment (start 127.748 116.668) (end 128.81 117.73) (width 0.2) (layer "B.Cu") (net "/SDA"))
 (segment (start 129.872 101.872) (end 129.872 113.089895) (width 0.2) (layer "B.Cu") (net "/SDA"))
 (segment (start 105.84 125.158) (end 104.69 124.008) (width 0.2) (layer "B.Cu") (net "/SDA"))
 (segment (start 127.748 114.750105) (end 127.748 116.668) (width 0.2) (layer "B.Cu") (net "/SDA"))
 (segment (start 138.43 88) (end 138.43 91.870429) (width 0.2) (layer "F.Cu") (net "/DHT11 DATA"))
 (segment (start 107.27 86.19) (end 113.08 92) (width 0.2) (layer "F.Cu") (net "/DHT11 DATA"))
 (segment (start 135.9 94.400429) (end 135.9 100.4) (width 0.2) (layer "F.Cu") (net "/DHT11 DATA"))
 (segment (start 138.43 91.870429) (end 135.9 94.400429) (width 0.2) (layer "F.Cu") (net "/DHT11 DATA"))
 (segment (start 135.9 100.4) (end 136.5 101) (width 0.2) (layer "F.Cu") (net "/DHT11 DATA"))
 (segment (start 100.08 86.19) (end 107.27 86.19) (width 0.2) (layer "F.Cu") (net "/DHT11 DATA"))
 (via (at 136.5 101) (size 0.6) (drill 0.3) (layers "F.Cu" "B.Cu") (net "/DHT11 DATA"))
 (segment (start 118.48 97.4) (end 113.08 92) (width 0.2) (layer "B.Cu") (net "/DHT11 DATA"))
 (segment (start 132.9 97.4) (end 118.48 97.4) (width 0.2) (layer "B.Cu") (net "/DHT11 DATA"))
 (segment (start 136.5 101) (end 132.9 97.4) (width 0.2) (layer "B.Cu") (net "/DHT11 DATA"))
 (segment (start 137.13 89.24) (end 135.89 88) (width 0.2) (layer "F.Cu") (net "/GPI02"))
 (segment (start 124.43 103.135256) (end 133.565256 94) (width 0.2) (layer "F.Cu") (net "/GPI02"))
 (segment (start 133.565256 94) (end 135.734744 94) (width 0.2) (layer "F.Cu") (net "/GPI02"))
 (segment (start 105.04 136.92) (end 105.04 134.659862) (width 0.2) (layer "F.Cu") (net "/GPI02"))
 (segment (start 124.43 115.269862) (end 124.43 103.135256) (width 0.2) (layer "F.Cu") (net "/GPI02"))
 (segment (start 105.04 134.659862) (end 124.43 115.269862) (width 0.2) (layer "F.Cu") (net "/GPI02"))
 (segment (start 135.734744 94) (end 137.13 92.604744) (width 0.2) (layer "F.Cu") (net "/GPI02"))
 (segment (start 137.13 92.604744) (end 137.13 89.24) (width 0.2) (layer "F.Cu") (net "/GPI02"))
 (segment (start 137.8 99.191358) (end 137.8 93.808642) (width 0.2) (layer "F.Cu") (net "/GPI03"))
 (segment (start 133.04 136.92) (end 142.27 127.69) (width 0.2) (layer "F.Cu") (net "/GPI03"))
 (segment (start 133.35 87.901358) (end 133.35 88) (width 0.2) (layer "F.Cu") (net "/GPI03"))
 (segment (start 141.808642 86.2) (end 135.051358 86.2) (width 0.2) (layer "F.Cu") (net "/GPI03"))
 (segment (start 142.27 127.69) (end 142.27 103.661358) (width 0.2) (layer "F.Cu") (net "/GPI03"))
 (segment (start 142.27 89.338642) (end 142.27 86.661358) (width 0.2) (layer "F.Cu") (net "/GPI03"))
 (segment (start 137.8 93.808642) (end 142.27 89.338642) (width 0.2) (layer "F.Cu") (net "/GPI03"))
 (segment (start 142.27 86.661358) (end 141.808642 86.2) (width 0.2) (layer "F.Cu") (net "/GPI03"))
 (segment (start 142.27 103.661358) (end 137.8 99.191358) (width 0.2) (layer "F.Cu") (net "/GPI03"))
 (segment (start 135.051358 86.2) (end 133.35 87.901358) (width 0.2) (layer "F.Cu") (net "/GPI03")))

